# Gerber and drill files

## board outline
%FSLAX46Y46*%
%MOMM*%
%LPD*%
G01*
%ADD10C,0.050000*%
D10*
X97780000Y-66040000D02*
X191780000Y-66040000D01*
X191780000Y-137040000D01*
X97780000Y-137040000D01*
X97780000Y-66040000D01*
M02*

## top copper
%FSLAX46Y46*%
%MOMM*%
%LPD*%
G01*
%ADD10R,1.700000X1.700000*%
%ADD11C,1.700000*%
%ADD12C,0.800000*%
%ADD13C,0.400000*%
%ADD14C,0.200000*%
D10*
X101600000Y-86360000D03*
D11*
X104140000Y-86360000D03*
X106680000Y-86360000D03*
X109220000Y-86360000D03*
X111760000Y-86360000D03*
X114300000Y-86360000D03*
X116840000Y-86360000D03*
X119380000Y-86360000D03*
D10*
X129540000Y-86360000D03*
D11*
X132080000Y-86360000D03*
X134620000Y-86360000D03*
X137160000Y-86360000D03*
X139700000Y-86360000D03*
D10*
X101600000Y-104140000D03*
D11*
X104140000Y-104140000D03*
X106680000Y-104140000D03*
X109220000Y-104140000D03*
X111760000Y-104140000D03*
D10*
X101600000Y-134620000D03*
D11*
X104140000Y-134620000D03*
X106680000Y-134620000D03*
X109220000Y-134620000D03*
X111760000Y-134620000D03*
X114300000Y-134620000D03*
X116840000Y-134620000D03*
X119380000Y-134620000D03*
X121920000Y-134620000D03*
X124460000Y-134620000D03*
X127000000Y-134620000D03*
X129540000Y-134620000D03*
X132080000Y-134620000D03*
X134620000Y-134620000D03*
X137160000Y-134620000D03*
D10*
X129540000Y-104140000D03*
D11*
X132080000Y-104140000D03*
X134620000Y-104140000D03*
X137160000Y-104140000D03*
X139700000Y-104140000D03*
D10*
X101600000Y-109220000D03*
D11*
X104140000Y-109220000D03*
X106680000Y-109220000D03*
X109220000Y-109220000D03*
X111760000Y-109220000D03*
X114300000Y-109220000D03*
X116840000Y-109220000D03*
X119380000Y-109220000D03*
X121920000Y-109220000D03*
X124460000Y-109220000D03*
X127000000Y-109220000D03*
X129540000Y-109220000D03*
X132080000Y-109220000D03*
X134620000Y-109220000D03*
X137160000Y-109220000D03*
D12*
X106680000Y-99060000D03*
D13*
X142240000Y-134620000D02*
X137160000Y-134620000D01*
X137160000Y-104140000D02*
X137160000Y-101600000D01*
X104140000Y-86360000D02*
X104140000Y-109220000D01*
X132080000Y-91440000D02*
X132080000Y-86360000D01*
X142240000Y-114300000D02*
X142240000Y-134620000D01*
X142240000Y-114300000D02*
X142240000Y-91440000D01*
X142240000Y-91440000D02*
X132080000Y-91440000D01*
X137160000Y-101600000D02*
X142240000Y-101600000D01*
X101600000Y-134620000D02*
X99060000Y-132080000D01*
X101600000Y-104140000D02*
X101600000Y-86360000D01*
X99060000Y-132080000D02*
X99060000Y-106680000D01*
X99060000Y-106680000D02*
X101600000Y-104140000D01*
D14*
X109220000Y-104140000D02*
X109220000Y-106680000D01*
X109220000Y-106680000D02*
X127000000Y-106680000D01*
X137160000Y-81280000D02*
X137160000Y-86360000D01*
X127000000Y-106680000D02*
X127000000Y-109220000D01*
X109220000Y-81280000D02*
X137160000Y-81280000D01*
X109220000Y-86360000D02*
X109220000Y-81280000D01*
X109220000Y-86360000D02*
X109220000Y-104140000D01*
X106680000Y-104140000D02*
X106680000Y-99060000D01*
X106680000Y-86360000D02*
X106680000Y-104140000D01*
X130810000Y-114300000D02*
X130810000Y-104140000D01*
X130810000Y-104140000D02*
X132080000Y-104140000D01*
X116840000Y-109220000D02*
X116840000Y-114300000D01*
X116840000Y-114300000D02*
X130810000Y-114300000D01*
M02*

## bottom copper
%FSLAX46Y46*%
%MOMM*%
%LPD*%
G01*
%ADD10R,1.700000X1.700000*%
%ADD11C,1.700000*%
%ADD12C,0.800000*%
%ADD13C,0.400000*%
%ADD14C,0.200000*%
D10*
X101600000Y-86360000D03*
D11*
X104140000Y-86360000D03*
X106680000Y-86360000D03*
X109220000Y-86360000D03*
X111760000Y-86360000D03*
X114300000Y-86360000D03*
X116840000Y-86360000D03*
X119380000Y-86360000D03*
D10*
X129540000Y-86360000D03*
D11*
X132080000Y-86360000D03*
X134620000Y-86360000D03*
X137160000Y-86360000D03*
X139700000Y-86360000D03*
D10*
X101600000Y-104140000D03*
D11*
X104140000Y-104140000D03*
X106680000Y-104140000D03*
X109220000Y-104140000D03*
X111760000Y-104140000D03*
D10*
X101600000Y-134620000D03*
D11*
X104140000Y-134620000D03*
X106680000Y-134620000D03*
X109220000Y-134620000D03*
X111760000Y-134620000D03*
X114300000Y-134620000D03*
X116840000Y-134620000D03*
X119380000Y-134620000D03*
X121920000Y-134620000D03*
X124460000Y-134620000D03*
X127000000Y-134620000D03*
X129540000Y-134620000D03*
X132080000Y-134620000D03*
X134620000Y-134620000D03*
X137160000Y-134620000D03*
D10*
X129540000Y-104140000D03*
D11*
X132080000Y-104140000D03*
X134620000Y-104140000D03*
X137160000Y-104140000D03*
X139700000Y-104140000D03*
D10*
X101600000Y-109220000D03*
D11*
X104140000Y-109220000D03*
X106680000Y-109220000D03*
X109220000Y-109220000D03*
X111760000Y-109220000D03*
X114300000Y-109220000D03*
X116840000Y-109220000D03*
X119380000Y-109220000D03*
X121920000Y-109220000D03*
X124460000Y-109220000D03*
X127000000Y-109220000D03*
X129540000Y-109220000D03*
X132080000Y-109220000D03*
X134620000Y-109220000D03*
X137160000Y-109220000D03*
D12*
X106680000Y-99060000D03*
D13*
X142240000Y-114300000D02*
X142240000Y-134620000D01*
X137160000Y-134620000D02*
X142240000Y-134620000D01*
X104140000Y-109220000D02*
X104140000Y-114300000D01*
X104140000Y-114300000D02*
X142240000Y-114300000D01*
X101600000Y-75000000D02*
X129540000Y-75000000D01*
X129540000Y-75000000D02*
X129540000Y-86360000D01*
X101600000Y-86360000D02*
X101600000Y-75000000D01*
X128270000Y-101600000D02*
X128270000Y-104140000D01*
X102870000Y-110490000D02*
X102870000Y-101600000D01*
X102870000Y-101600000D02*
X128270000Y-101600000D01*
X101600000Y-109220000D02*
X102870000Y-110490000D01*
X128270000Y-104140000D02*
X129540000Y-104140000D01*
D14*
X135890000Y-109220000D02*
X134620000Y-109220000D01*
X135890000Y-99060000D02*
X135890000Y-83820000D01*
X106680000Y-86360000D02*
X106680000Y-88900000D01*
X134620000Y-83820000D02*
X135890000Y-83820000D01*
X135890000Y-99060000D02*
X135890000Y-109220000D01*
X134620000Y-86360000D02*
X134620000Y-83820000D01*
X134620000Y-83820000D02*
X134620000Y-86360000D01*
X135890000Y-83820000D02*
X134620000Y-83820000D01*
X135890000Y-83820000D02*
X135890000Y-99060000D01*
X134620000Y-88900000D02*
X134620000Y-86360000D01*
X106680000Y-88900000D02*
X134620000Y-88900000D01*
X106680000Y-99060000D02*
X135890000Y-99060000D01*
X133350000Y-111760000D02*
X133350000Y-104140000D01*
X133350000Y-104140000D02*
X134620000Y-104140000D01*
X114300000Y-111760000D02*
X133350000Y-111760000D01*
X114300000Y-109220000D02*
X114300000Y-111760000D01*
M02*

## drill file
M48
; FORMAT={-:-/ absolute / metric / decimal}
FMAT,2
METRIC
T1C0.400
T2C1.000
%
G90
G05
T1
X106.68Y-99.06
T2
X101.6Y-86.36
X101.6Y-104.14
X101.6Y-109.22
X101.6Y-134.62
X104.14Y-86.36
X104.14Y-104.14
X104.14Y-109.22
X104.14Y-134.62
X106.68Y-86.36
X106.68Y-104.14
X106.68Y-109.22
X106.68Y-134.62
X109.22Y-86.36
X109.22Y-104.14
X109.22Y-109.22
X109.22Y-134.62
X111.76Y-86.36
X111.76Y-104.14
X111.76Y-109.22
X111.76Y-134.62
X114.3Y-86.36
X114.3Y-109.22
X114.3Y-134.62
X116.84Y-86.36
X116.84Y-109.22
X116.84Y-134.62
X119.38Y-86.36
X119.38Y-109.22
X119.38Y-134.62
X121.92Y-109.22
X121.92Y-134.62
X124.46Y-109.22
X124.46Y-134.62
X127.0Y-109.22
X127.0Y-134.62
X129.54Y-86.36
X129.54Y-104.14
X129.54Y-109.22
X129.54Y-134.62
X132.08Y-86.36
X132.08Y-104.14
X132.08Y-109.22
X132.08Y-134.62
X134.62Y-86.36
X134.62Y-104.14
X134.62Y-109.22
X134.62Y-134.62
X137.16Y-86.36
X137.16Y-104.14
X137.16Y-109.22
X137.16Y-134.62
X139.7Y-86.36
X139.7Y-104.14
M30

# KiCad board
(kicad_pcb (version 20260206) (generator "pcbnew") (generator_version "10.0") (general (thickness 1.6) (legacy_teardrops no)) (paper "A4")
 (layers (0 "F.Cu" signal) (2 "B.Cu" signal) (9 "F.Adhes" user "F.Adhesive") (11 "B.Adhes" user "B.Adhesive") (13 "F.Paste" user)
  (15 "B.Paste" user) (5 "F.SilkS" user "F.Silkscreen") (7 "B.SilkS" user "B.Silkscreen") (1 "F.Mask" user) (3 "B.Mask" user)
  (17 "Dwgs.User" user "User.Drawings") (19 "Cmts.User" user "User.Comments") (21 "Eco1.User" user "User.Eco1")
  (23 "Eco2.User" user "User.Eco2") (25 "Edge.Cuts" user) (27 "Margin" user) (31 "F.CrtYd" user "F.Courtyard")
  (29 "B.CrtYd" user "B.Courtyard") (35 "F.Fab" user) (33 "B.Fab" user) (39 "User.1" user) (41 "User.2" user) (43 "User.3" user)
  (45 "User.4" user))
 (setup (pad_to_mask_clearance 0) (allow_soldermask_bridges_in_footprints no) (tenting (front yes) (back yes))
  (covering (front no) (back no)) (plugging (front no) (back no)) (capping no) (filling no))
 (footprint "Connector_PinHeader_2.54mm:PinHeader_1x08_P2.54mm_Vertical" (layer "F.Cu") (at 101.6 86.36 90)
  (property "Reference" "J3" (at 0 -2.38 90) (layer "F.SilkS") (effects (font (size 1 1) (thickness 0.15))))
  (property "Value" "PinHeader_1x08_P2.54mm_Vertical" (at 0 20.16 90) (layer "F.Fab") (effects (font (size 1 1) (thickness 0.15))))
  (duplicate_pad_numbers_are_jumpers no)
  (pad "1" thru_hole rect (at 0 0 90) (size 1.7 1.7) (drill 1) (layers "*.Cu" "*.Mask") (remove_unused_layers no) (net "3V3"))
  (pad "2" thru_hole circle (at 0 2.54 90) (size 1.7 1.7) (drill 1) (layers "*.Cu" "*.Mask") (remove_unused_layers no) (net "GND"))
  (pad "3" thru_hole circle (at 0 5.08 90) (size 1.7 1.7) (drill 1) (layers "*.Cu" "*.Mask") (remove_unused_layers no) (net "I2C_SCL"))
  (pad "4" thru_hole circle (at 0 7.62 90) (size 1.7 1.7) (drill 1) (layers "*.Cu" "*.Mask") (remove_unused_layers no) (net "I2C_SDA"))
  (pad "5" thru_hole circle (at 0 10.16 90) (size 1.7 1.7) (drill 1) (layers "*.Cu" "*.Mask") (remove_unused_layers no) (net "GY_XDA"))
  (pad "6" thru_hole circle (at 0 12.7 90) (size 1.7 1.7) (drill 1) (layers "*.Cu" "*.Mask") (remove_unused_layers no) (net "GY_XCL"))
  (pad "7" thru_hole circle (at 0 15.24 90) (size 1.7 1.7) (drill 1) (layers "*.Cu" "*.Mask") (remove_unused_layers no) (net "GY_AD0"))
  (pad "8" thru_hole circle (at 0 17.78 90) (size 1.7 1.7) (drill 1) (layers "*.Cu" "*.Mask") (remove_unused_layers no) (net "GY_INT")))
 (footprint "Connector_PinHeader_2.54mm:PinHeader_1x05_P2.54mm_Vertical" (layer "F.Cu") (at 129.54 86.36 90)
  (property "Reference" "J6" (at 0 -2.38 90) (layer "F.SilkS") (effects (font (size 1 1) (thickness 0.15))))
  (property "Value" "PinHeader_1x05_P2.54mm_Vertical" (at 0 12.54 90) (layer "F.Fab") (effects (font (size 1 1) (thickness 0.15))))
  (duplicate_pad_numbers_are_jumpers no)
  (pad "1" thru_hole rect (at 0 0 90) (size 1.7 1.7) (drill 1) (layers "*.Cu" "*.Mask") (remove_unused_layers no) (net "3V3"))
  (pad "2" thru_hole circle (at 0 2.54 90) (size 1.7 1.7) (drill 1) (layers "*.Cu" "*.Mask") (remove_unused_layers no) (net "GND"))
  (pad "3" thru_hole circle (at 0 5.08 90) (size 1.7 1.7) (drill 1) (layers "*.Cu" "*.Mask") (remove_unused_layers no) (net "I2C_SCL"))
  (pad "4" thru_hole circle (at 0 7.62 90) (size 1.7 1.7) (drill 1) (layers "*.Cu" "*.Mask") (remove_unused_layers no) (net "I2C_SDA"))
  (pad "5" thru_hole circle (at 0 10.16 90) (size 1.7 1.7) (drill 1) (layers "*.Cu" "*.Mask") (remove_unused_layers no) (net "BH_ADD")))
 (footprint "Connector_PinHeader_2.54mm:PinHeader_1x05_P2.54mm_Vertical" (layer "F.Cu") (at 101.6 104.14 90)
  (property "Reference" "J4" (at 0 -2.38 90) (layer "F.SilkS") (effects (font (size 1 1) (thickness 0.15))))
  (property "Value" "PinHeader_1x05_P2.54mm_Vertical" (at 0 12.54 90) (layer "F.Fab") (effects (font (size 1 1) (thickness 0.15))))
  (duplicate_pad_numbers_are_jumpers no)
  (pad "1" thru_hole rect (at 0 0 90) (size 1.7 1.7) (drill 1) (layers "*.Cu" "*.Mask") (remove_unused_layers no) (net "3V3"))
  (pad "2" thru_hole circle (at 0 2.54 90) (size 1.7 1.7) (drill 1) (layers "*.Cu" "*.Mask") (remove_unused_layers no) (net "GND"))
  (pad "3" thru_hole circle (at 0 5.08 90) (size 1.7 1.7) (drill 1) (layers "*.Cu" "*.Mask") (remove_unused_layers no) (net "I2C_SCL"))
  (pad "4" thru_hole circle (at 0 7.62 90) (size 1.7 1.7) (drill 1) (layers "*.Cu" "*.Mask") (remove_unused_layers no) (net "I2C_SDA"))
  (pad "5" thru_hole circle (at 0 10.16 90) (size 1.7 1.7) (drill 1) (layers "*.Cu" "*.Mask") (remove_unused_layers no) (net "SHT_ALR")))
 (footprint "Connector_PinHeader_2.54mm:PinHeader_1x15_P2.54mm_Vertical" (layer "F.Cu") (at 101.6 134.62 90)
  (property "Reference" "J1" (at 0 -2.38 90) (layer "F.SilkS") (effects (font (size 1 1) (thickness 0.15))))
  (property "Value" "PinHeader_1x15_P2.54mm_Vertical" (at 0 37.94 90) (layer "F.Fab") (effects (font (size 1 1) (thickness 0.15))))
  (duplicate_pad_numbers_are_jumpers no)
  (pad "1" thru_hole rect (at 0 0 90) (size 1.7 1.7) (drill 1) (layers "*.Cu" "*.Mask") (remove_unused_layers no) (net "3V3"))
  (pad "2" thru_hole circle (at 0 2.54 90) (size 1.7 1.7) (drill 1) (layers "*.Cu" "*.Mask") (remove_unused_layers no) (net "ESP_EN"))
  (pad "3" thru_hole circle (at 0 5.08 90) (size 1.7 1.7) (drill 1) (layers "*.Cu" "*.Mask") (remove_unused_layers no) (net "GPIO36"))
  (pad "4" thru_hole circle (at 0 7.62 90) (size 1.7 1.7) (drill 1) (layers "*.Cu" "*.Mask") (remove_unused_layers no) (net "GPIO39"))
  (pad "5" thru_hole circle (at 0 10.16 90) (size 1.7 1.7) (drill 1) (layers "*.Cu" "*.Mask") (remove_unused_layers no) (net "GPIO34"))
  (pad "6" thru_hole circle (at 0 12.7 90) (size 1.7 1.7) (drill 1) (layers "*.Cu" "*.Mask") (remove_unused_layers no) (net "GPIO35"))
  (pad "7" thru_hole circle (at 0 15.24 90) (size 1.7 1.7) (drill 1) (layers "*.Cu" "*.Mask") (remove_unused_layers no) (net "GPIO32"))
  (pad "8" thru_hole circle (at 0 17.78 90) (size 1.7 1.7) (drill 1) (layers "*.Cu" "*.Mask") (remove_unused_layers no) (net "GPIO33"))
  (pad "9" thru_hole circle (at 0 20.32 90) (size 1.7 1.7) (drill 1) (layers "*.Cu" "*.Mask") (remove_unused_layers no) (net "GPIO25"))
  (pad "10" thru_hole circle (at 0 22.86 90) (size 1.7 1.7) (drill 1) (layers "*.Cu" "*.Mask") (remove_unused_layers no) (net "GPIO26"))
  (pad "11" thru_hole circle (at 0 25.4 90) (size 1.7 1.7) (drill 1) (layers "*.Cu" "*.Mask") (remove_unused_layers no) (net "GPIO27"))
  (pad "12" thru_hole circle (at 0 27.94 90) (size 1.7 1.7) (drill 1) (layers "*.Cu" "*.Mask") (remove_unused_layers no) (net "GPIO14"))
  (pad "13" thru_hole circle (at 0 30.48 90) (size 1.7 1.7) (drill 1) (layers "*.Cu" "*.Mask") (remove_unused_layers no) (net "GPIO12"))
  (pad "14" thru_hole circle (at 0 33.02 90) (size 1.7 1.7) (drill 1) (layers "*.Cu" "*.Mask") (remove_unused_layers no) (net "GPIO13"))
  (pad "15" thru_hole circle (at 0 35.56 90) (size 1.7 1.7) (drill 1) (layers "*.Cu" "*.Mask") (remove_unused_layers no) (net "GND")))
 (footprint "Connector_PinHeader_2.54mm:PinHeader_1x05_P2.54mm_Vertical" (layer "F.Cu") (at 129.54 104.14 90)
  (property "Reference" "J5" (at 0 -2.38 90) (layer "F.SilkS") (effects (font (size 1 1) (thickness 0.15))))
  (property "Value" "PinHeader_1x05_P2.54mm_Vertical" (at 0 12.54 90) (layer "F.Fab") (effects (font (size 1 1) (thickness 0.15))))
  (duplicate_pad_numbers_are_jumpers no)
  (pad "1" thru_hole rect (at 0 0 90) (size 1.7 1.7) (drill 1) (layers "*.Cu" "*.Mask") (remove_unused_layers no) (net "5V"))
  (pad "2" thru_hole circle (at 0 2.54 90) (size 1.7 1.7) (drill 1) (layers "*.Cu" "*.Mask") (remove_unused_layers no) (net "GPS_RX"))
  (pad "3" thru_hole circle (at 0 5.08 90) (size 1.7 1.7) (drill 1) (layers "*.Cu" "*.Mask") (remove_unused_layers no) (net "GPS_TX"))
  (pad "4" thru_hole circle (at 0 7.62 90) (size 1.7 1.7) (drill 1) (layers "*.Cu" "*.Mask") (remove_unused_layers no) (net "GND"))
  (pad "5" thru_hole circle (at 0 10.16 90) (size 1.7 1.7) (drill 1) (layers "*.Cu" "*.Mask") (remove_unused_layers no) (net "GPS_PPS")))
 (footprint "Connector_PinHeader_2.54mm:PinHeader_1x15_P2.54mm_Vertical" (layer "F.Cu") (at 101.6 109.22 90)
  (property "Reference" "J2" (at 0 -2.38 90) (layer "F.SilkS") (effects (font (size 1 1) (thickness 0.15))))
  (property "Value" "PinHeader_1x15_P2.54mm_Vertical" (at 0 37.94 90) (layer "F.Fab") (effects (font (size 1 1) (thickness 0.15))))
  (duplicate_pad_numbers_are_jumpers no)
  (pad "1" thru_hole rect (at 0 0 90) (size 1.7 1.7) (drill 1) (layers "*.Cu" "*.Mask") (remove_unused_layers no) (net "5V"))
  (pad "2" thru_hole circle (at 0 2.54 90) (size 1.7 1.7) (drill 1) (layers "*.Cu" "*.Mask") (remove_unused_layers no) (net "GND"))
  (pad "3" thru_hole circle (at 0 5.08 90) (size 1.7 1.7) (drill 1) (layers "*.Cu" "*.Mask") (remove_unused_layers no) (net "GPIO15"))
  (pad "4" thru_hole circle (at 0 7.62 90) (size 1.7 1.7) (drill 1) (layers "*.Cu" "*.Mask") (remove_unused_layers no) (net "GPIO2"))
  (pad "5" thru_hole circle (at 0 10.16 90) (size 1.7 1.7) (drill 1) (layers "*.Cu" "*.Mask") (remove_unused_layers no) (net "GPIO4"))
  (pad "6" thru_hole circle (at 0 12.7 90) (size 1.7 1.7) (drill 1) (layers "*.Cu" "*.Mask") (remove_unused_layers no) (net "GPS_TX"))
  (pad "7" thru_hole circle (at 0 15.24 90) (size 1.7 1.7) (drill 1) (layers "*.Cu" "*.Mask") (remove_unused_layers no) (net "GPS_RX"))
  (pad "8" thru_hole circle (at 0 17.78 90) (size 1.7 1.7) (drill 1) (layers "*.Cu" "*.Mask") (remove_unused_layers no) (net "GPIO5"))
  (pad "9" thru_hole circle (at 0 20.32 90) (size 1.7 1.7) (drill 1) (layers "*.Cu" "*.Mask") (remove_unused_layers no) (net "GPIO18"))
  (pad "10" thru_hole circle (at 0 22.86 90) (size 1.7 1.7) (drill 1) (layers "*.Cu" "*.Mask") (remove_unused_layers no) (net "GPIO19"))
  (pad "11" thru_hole circle (at 0 25.4 90) (size 1.7 1.7) (drill 1) (layers "*.Cu" "*.Mask") (remove_unused_layers no) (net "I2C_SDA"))
  (pad "12" thru_hole circle (at 0 27.94 90) (size 1.7 1.7) (drill 1) (layers "*.Cu" "*.Mask") (remove_unused_layers no) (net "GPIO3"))
  (pad "13" thru_hole circle (at 0 30.48 90) (size 1.7 1.7) (drill 1) (layers "*.Cu" "*.Mask") (remove_unused_layers no) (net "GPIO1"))
  (pad "14" thru_hole circle (at 0 33.02 90) (size 1.7 1.7) (drill 1) (layers "*.Cu" "*.Mask") (remove_unused_layers no) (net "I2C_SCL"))
  (pad "15" thru_hole circle (at 0 35.56 90) (size 1.7 1.7) (drill 1) (layers "*.Cu" "*.Mask") (remove_unused_layers no) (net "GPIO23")))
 (gr_rect (start 97.78 66.04) (end 191.78 137.04) (stroke (width 0.05) (type solid)) (fill no) (layer "Edge.Cuts"))
 (segment (start 142.24 134.62) (end 137.16 134.62) (width 0.4) (layer "F.Cu") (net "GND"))
 (segment (start 137.16 104.14) (end 137.16 101.6) (width 0.4) (layer "F.Cu") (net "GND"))
 (segment (start 104.14 86.36) (end 104.14 109.22) (width 0.4) (layer "F.Cu") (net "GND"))
 (segment (start 132.08 91.44) (end 132.08 86.36) (width 0.4) (layer "F.Cu") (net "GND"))
 (segment (start 142.24 114.3) (end 142.24 134.62) (width 0.4) (layer "F.Cu") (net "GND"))
 (segment (start 142.24 114.3) (end 142.24 91.44) (width 0.4) (layer "F.Cu") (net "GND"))
 (segment (start 142.24 91.44) (end 132.08 91.44) (width 0.4) (layer "F.Cu") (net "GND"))
 (segment (start 137.16 101.6) (end 142.24 101.6) (width 0.4) (layer "F.Cu") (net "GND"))
 (segment (start 142.24 114.3) (end 142.24 134.62) (width 0.4) (layer "B.Cu") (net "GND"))
 (segment (start 137.16 134.62) (end 142.24 134.62) (width 0.4) (layer "B.Cu") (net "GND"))
 (segment (start 104.14 109.22) (end 104.14 114.3) (width 0.4) (layer "B.Cu") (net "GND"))
 (segment (start 104.14 114.3) (end 142.24 114.3) (width 0.4) (layer "B.Cu") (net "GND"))
 (segment (start 101.6 134.62) (end 99.06 132.08) (width 0.4) (layer "F.Cu") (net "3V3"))
 (segment (start 101.6 104.14) (end 101.6 86.36) (width 0.4) (layer "F.Cu") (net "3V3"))
 (segment (start 99.06 132.08) (end 99.06 106.68) (width 0.4) (layer "F.Cu") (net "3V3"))
 (segment (start 99.06 106.68) (end 101.6 104.14) (width 0.4) (layer "F.Cu") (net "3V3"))
 (segment (start 101.6 75) (end 129.54 75) (width 0.4) (layer "B.Cu") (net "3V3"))
 (segment (start 129.54 75) (end 129.54 86.36) (width 0.4) (layer "B.Cu") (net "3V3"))
 (segment (start 101.6 86.36) (end 101.6 75) (width 0.4) (layer "B.Cu") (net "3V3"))
 (segment (start 128.27 101.6) (end 128.27 104.14) (width 0.4) (layer "B.Cu") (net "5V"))
 (segment (start 102.87 110.49) (end 102.87 101.6) (width 0.4) (layer "B.Cu") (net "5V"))
 (segment (start 102.87 101.6) (end 128.27 101.6) (width 0.4) (layer "B.Cu") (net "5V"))
 (segment (start 101.6 109.22) (end 102.87 110.49) (width 0.4) (layer "B.Cu") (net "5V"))
 (segment (start 128.27 104.14) (end 129.54 104.14) (width 0.4) (layer "B.Cu") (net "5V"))
 (segment (start 109.22 104.14) (end 109.22 106.68) (width 0.2) (layer "F.Cu") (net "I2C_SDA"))
 (segment (start 109.22 106.68) (end 127 106.68) (width 0.2) (layer "F.Cu") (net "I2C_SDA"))
 (segment (start 137.16 81.28) (end 137.16 86.36) (width 0.2) (layer "F.Cu") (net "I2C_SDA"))
 (segment (start 127 106.68) (end 127 109.22) (width 0.2) (layer "F.Cu") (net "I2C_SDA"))
 (segment (start 109.22 81.28) (end 137.16 81.28) (width 0.2) (layer "F.Cu") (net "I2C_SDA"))
 (segment (start 109.22 86.36) (end 109.22 81.28) (width 0.2) (layer "F.Cu") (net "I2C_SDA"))
 (segment (start 109.22 86.36) (end 109.22 104.14) (width 0.2) (layer "F.Cu") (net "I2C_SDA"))
 (segment (start 106.68 104.14) (end 106.68 99.06) (width 0.2) (layer "F.Cu") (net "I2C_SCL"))
 (segment (start 106.68 86.36) (end 106.68 104.14) (width 0.2) (layer "F.Cu") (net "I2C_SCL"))
 (via (at 106.68 99.06) (size 0.8) (drill 0.4) (layers "F.Cu" "B.Cu") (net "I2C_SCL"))
 (segment (start 135.89 109.22) (end 134.62 109.22) (width 0.2) (layer "B.Cu") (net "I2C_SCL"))
 (segment (start 135.89 99.06) (end 135.89 83.82) (width 0.2) (layer "B.Cu") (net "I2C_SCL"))
 (segment (start 106.68 86.36) (end 106.68 88.9) (width 0.2) (layer "B.Cu") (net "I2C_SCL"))
 (segment (start 134.62 83.82) (end 135.89 83.82) (width 0.2) (layer "B.Cu") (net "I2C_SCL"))
 (segment (start 135.89 99.06) (end 135.89 109.22) (width 0.2) (layer "B.Cu") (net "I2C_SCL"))
 (segment (start 134.62 86.36) (end 134.62 83.82) (width 0.2) (layer "B.Cu") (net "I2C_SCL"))
 (segment (start 134.62 83.82) (end 134.62 86.36) (width 0.2) (layer "B.Cu") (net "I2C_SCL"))
 (segment (start 135.89 83.82) (end 134.62 83.82) (width 0.2) (layer "B.Cu") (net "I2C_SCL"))
 (segment (start 135.89 83.82) (end 135.89 99.06) (width 0.2) (layer "B.Cu") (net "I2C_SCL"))
 (segment (start 134.62 88.9) (end 134.62 86.36) (width 0.2) (layer "B.Cu") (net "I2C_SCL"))
 (segment (start 106.68 88.9) (end 134.62 88.9) (width 0.2) (layer "B.Cu") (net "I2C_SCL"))
 (segment (start 106.68 99.06) (end 135.89 99.06) (width 0.2) (layer "B.Cu") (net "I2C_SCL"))
 (segment (start 130.81 114.3) (end 130.81 104.14) (width 0.2) (layer "F.Cu") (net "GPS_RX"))
 (segment (start 130.81 104.14) (end 132.08 104.14) (width 0.2) (layer "F.Cu") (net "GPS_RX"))
 (segment (start 116.84 109.22) (end 116.84 114.3) (width 0.2) (layer "F.Cu") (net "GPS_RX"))
 (segment (start 116.84 114.3) (end 130.81 114.3) (width 0.2) (layer "F.Cu") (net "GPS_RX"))
 (segment (start 133.35 111.76) (end 133.35 104.14) (width 0.2) (layer "B.Cu") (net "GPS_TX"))
 (segment (start 133.35 104.14) (end 134.62 104.14) (width 0.2) (layer "B.Cu") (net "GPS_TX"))
 (segment (start 114.3 111.76) (end 133.35 111.76) (width 0.2) (layer "B.Cu") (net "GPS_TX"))
 (segment (start 114.3 109.22) (end 114.3 111.76) (width 0.2) (layer "B.Cu") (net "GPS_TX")))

